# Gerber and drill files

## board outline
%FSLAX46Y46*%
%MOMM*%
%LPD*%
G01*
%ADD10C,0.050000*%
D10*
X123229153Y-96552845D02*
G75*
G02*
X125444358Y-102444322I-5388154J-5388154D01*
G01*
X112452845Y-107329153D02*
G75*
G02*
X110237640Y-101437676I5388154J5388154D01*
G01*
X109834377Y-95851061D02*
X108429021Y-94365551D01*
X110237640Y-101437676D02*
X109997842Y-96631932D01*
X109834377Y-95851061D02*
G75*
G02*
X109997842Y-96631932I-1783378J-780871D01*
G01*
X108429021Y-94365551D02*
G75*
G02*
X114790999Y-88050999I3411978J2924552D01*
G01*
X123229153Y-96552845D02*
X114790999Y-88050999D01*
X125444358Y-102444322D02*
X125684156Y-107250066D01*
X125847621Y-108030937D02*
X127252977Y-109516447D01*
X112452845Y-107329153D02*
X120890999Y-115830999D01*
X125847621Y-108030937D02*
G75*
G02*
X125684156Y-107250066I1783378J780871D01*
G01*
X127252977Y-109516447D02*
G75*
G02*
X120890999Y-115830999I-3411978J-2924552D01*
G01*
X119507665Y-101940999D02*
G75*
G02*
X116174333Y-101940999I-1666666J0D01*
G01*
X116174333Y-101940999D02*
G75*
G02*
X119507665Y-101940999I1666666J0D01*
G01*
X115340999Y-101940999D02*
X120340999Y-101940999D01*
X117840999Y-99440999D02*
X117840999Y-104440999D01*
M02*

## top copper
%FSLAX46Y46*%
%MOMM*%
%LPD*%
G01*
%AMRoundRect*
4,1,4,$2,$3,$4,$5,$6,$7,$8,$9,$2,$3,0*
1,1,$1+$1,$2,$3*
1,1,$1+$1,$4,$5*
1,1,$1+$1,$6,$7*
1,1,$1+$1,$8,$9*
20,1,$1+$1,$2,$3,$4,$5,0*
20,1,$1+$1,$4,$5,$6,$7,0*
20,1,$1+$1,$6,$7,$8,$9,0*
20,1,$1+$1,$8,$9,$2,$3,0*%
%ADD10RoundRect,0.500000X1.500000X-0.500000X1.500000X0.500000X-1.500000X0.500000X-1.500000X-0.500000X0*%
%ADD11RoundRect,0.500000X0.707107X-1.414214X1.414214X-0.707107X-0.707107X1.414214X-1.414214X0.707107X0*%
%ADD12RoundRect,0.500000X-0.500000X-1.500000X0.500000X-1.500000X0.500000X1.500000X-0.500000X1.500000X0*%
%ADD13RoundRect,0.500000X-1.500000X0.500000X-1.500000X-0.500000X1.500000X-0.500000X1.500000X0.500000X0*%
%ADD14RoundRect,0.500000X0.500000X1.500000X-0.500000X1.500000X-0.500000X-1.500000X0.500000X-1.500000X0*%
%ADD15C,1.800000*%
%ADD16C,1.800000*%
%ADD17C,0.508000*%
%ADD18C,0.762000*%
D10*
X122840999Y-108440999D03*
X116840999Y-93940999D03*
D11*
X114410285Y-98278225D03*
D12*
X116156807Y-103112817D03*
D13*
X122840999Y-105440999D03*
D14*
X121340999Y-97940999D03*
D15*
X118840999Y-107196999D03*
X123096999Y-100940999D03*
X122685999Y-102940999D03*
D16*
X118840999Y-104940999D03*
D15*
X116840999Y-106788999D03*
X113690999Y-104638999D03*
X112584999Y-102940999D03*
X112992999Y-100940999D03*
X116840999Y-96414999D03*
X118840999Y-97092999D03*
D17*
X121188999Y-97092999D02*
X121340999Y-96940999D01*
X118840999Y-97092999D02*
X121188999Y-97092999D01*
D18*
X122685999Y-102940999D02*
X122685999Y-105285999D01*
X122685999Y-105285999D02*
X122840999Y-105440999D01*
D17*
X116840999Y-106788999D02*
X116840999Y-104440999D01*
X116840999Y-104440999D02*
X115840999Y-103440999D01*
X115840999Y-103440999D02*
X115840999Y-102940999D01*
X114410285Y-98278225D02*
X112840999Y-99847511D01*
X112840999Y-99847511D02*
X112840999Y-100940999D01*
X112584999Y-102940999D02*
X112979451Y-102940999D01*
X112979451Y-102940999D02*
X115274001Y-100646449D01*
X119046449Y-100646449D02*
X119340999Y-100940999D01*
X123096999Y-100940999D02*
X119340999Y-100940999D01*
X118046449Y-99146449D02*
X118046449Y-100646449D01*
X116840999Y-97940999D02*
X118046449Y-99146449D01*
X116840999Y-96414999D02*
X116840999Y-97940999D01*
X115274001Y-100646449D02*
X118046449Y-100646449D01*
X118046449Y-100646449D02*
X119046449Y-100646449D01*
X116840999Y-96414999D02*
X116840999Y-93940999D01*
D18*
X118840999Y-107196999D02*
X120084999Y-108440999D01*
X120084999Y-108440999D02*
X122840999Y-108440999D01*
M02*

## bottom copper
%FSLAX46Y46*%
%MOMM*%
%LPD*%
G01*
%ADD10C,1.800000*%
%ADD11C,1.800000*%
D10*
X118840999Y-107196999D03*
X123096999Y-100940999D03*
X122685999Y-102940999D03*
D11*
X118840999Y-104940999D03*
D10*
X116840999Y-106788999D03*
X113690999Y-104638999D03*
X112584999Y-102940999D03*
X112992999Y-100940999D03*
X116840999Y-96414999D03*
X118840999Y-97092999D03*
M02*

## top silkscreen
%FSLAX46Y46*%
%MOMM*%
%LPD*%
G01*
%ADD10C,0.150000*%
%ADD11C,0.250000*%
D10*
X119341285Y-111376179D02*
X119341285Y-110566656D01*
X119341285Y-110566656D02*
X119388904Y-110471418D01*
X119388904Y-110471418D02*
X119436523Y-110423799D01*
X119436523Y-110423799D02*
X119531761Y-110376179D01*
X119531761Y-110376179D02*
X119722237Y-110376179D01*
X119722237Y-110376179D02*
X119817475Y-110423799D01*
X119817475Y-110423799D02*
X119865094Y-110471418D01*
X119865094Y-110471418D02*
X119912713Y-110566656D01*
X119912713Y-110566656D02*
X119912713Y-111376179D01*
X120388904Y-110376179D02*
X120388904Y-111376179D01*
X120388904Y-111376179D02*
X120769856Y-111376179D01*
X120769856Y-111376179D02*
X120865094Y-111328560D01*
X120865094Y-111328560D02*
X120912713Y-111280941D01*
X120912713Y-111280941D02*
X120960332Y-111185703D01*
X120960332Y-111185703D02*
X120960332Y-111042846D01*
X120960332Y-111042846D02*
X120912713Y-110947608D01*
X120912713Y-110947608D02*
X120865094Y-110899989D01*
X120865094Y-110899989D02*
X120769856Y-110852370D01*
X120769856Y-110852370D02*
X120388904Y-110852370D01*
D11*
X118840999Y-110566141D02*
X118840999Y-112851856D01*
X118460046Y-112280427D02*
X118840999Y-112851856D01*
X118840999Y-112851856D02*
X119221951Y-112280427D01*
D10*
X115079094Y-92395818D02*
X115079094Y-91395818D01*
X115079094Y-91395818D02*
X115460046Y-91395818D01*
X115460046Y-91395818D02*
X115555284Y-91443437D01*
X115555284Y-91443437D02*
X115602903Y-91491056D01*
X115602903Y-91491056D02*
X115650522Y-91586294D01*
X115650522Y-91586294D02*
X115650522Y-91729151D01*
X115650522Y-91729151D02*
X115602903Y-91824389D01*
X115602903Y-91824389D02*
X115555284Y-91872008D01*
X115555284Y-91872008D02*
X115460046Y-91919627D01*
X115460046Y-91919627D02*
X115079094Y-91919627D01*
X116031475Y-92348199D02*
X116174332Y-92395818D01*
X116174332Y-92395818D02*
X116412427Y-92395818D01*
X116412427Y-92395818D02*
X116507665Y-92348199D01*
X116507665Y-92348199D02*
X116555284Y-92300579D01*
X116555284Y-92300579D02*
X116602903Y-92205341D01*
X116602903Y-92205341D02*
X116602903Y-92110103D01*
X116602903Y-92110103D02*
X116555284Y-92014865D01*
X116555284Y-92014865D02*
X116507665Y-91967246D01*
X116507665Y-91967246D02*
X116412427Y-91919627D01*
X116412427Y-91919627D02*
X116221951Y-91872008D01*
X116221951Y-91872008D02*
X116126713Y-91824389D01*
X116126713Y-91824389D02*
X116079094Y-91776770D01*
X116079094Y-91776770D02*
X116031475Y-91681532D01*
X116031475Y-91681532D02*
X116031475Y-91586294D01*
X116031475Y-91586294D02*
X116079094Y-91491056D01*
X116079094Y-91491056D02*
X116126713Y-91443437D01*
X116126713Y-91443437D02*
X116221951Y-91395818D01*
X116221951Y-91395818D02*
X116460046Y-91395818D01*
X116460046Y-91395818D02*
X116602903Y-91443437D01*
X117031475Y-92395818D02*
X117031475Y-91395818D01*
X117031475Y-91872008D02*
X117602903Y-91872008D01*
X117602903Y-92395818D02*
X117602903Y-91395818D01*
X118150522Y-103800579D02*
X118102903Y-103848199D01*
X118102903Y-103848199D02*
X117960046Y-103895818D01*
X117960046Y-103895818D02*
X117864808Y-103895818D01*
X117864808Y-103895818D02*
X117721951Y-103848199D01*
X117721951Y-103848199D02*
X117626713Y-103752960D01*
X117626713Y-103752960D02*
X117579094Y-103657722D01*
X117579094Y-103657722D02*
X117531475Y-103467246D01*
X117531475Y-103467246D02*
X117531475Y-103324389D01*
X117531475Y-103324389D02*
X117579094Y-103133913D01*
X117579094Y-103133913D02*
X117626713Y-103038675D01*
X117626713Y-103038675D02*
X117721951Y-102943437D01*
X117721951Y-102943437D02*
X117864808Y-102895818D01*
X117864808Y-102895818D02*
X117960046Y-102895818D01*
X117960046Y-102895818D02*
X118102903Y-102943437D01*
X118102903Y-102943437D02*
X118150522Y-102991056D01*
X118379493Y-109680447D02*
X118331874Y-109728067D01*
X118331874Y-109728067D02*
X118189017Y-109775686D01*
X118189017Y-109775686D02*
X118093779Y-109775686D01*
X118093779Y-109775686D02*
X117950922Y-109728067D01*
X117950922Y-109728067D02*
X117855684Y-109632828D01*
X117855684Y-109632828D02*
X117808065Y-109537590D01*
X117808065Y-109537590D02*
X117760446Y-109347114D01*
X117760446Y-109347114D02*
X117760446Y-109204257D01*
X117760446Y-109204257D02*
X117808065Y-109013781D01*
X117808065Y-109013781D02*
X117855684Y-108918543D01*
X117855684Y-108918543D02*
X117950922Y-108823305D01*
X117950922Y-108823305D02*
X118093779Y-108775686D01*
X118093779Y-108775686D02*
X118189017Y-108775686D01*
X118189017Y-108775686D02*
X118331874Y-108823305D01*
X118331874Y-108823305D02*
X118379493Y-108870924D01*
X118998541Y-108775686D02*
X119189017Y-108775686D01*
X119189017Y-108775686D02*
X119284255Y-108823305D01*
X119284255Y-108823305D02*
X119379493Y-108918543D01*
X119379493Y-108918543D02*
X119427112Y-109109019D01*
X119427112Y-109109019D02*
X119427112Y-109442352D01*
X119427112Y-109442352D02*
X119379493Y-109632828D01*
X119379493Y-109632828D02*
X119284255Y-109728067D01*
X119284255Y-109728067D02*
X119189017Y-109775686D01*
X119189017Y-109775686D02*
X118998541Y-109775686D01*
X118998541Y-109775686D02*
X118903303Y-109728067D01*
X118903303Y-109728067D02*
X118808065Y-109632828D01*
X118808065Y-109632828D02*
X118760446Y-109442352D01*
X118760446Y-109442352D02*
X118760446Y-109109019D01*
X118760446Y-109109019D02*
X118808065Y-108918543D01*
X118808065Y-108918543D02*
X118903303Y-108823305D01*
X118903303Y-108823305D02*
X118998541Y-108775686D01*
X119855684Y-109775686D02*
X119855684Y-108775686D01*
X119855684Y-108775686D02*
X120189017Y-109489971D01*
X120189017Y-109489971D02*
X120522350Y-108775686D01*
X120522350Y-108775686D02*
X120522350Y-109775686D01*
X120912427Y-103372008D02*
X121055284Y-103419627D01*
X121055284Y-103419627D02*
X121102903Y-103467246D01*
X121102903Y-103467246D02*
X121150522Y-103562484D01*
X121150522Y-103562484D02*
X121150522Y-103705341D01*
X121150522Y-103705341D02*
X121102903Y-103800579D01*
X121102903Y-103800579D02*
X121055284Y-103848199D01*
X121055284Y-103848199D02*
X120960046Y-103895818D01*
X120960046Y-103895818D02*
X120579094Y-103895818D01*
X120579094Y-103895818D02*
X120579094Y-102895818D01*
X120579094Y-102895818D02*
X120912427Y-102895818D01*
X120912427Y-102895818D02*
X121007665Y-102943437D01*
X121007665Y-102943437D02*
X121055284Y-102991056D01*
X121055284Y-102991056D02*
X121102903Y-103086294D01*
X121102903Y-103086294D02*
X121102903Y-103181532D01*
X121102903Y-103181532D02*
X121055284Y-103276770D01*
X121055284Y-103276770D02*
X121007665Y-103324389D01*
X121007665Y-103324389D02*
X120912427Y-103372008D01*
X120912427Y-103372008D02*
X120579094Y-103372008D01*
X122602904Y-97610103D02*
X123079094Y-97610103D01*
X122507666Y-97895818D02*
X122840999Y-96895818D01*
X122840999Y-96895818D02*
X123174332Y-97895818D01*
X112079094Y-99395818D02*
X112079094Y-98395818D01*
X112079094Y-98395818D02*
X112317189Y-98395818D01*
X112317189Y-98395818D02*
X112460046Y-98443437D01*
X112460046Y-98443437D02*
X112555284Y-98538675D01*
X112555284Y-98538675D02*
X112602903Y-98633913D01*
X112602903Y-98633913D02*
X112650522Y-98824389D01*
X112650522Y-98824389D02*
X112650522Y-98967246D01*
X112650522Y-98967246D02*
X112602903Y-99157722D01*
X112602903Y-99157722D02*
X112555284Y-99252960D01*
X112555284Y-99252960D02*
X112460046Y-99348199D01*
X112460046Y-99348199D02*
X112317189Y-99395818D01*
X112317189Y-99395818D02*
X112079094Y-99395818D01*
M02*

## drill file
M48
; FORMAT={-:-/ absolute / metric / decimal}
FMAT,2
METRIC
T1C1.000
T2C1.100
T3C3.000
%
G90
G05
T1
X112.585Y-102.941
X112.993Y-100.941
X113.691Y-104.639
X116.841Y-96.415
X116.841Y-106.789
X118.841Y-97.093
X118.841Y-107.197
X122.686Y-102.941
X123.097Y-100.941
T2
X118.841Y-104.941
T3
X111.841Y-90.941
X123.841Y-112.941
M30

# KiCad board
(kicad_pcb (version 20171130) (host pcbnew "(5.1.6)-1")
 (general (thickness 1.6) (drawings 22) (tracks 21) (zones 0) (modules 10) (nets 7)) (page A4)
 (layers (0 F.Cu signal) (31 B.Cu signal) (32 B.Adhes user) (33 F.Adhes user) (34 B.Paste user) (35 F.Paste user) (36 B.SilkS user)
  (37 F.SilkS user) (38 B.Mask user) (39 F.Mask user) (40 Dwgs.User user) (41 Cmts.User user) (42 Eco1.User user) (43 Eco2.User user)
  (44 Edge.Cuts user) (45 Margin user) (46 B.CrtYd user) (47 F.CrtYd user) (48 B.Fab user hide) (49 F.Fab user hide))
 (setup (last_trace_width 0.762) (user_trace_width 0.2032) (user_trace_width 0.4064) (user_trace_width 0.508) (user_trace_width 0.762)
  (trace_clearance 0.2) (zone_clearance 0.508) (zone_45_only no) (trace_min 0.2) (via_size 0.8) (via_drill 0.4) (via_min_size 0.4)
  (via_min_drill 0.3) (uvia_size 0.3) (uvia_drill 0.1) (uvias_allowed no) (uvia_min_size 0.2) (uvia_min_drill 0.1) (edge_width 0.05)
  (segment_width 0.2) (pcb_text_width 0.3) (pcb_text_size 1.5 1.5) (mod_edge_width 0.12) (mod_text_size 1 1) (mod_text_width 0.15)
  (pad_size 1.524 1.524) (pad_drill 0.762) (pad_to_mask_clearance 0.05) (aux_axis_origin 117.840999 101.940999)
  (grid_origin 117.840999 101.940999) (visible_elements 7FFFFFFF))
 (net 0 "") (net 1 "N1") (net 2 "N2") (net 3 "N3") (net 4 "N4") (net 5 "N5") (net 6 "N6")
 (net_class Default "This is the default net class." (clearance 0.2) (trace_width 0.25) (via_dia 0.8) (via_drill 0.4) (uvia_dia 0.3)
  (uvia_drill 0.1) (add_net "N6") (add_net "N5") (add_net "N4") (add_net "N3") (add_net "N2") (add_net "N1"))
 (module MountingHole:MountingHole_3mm (layer B.Cu) (at 111.840999 90.940999 180)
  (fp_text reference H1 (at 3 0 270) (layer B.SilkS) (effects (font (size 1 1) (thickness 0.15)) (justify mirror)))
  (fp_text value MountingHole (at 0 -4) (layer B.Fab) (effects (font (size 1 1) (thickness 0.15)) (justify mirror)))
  (pad 1 np_thru_hole circle (at 0 0 180) (size 3 3) (drill 3) (layers *.Cu *.Mask)))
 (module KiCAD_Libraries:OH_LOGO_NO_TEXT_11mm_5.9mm (layer B.Cu) (at 118.340999 101.440999 200)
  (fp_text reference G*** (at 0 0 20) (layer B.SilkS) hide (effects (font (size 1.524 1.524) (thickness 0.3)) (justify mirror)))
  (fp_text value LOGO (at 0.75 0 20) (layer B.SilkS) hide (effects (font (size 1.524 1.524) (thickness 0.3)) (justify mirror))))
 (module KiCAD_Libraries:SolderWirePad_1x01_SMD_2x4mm (layer F.Cu) (at 122.840999 108.440999 90)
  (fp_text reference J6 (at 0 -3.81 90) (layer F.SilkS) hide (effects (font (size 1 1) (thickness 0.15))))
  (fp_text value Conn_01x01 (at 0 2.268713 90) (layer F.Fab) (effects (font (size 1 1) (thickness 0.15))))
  (pad 1 smd roundrect (at 0 0 90) (size 2 4) (layers F.Cu F.Paste F.Mask) (roundrect_rratio 0.25) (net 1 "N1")))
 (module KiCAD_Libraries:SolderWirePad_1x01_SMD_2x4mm (layer F.Cu) (at 116.840999 93.940999 90)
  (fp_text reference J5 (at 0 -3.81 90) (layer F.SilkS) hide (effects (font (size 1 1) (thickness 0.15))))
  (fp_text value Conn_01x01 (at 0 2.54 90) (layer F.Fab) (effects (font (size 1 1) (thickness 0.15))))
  (pad 1 smd roundrect (at 0 0 90) (size 2 4) (layers F.Cu F.Paste F.Mask) (roundrect_rratio 0.25) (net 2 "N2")))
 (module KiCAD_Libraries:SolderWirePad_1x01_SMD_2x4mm (layer F.Cu) (at 114.410285 98.278225 45)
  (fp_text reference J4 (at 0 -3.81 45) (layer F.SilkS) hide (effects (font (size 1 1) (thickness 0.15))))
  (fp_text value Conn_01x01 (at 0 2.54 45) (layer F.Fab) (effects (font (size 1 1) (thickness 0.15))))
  (pad 1 smd roundrect (at 0 0 45) (size 2 4) (layers F.Cu F.Paste F.Mask) (roundrect_rratio 0.25) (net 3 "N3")))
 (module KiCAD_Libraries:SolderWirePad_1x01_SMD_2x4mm (layer F.Cu) (at 116.156807 103.112817)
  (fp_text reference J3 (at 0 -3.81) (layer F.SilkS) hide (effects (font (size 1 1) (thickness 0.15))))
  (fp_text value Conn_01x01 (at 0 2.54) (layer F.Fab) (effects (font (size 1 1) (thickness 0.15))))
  (pad 1 smd roundrect (at 0 0) (size 2 4) (layers F.Cu F.Paste F.Mask) (roundrect_rratio 0.25) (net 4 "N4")))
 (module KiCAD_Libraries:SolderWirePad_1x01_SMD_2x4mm (layer F.Cu) (at 122.840999 105.440999 270)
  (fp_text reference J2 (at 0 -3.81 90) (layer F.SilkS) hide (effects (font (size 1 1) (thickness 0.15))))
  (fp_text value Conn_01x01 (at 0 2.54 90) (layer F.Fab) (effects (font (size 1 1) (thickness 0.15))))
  (pad 1 smd roundrect (at 0 0 270) (size 2 4) (layers F.Cu F.Paste F.Mask) (roundrect_rratio 0.25) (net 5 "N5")))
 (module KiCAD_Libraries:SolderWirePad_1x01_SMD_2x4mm (layer F.Cu) (at 121.340999 97.940999 180)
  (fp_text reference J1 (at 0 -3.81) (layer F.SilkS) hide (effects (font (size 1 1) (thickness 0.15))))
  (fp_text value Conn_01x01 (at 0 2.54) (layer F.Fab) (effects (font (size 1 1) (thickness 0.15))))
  (pad 1 smd roundrect (at 0 0 180) (size 2 4) (layers F.Cu F.Paste F.Mask) (roundrect_rratio 0.25) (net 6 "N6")))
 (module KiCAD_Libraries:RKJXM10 (layer B.Cu) (at 117.840999 101.940999)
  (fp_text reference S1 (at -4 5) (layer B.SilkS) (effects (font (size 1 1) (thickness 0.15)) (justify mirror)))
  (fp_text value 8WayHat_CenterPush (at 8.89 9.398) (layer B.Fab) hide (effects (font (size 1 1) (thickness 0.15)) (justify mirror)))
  (pad COM thru_hole circle (at 1 5.256) (size 1.8 1.8) (drill 1) (layers *.Cu *.Mask) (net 1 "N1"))
  (pad PUSH3 thru_hole circle (at 5.256 -1) (size 1.8 1.8) (drill 1) (layers *.Cu *.Mask) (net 2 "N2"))
  (pad B thru_hole circle (at 4.845 1) (size 1.8 1.8) (drill 1) (layers *.Cu *.Mask) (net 5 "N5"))
  (pad "" np_thru_hole circle (at 1 3) (size 1.8 1.8) (drill 1.1) (layers *.Cu *.Mask))
  (pad C thru_hole circle (at -1 4.848) (size 1.8 1.8) (drill 1) (layers *.Cu *.Mask) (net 4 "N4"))
  (pad GND thru_hole circle (at -4.15 2.698) (size 1.8 1.8) (drill 1) (layers *.Cu *.Mask))
  (pad PUSH1 thru_hole circle (at -5.256 1) (size 1.8 1.8) (drill 1) (layers *.Cu *.Mask) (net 2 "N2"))
  (pad D thru_hole circle (at -4.848 -1) (size 1.8 1.8) (drill 1) (layers *.Cu *.Mask) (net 3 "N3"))
  (pad PUSH2 thru_hole circle (at -1 -5.526) (size 1.8 1.8) (drill 1) (layers *.Cu *.Mask) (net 2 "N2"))
  (pad A thru_hole circle (at 1 -4.848) (size 1.8 1.8) (drill 1) (layers *.Cu *.Mask) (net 6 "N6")))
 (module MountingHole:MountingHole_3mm (layer B.Cu) (at 123.840999 112.940999)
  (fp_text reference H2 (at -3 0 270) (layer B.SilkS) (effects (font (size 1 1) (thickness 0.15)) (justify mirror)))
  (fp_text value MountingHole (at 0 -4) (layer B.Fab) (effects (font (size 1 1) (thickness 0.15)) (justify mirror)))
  (pad 1 np_thru_hole circle (at 0 0) (size 3 3) (drill 3) (layers *.Cu *.Mask)))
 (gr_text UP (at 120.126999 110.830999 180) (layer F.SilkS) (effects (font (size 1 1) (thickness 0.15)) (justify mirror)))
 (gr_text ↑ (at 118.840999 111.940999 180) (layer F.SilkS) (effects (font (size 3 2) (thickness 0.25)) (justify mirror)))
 (gr_arc (start 117.840999 101.940999) (end 125.444358 102.444322) (angle -48.787309) (layer Edge.Cuts) (width 0.05))
 (gr_arc (start 117.840999 101.940999) (end 110.23764 101.437676) (angle -48.787309) (layer Edge.Cuts) (width 0.05))
 (gr_line (start 109.834377 95.851061) (end 108.429021 94.365551) (layer Edge.Cuts) (width 0.05))
 (gr_line (start 110.23764 101.437676) (end 109.997842 96.631932) (layer Edge.Cuts) (width 0.05))
 (gr_arc (start 108.050999 96.631932) (end 109.997842 96.631932) (angle -23.64670356) (layer Edge.Cuts) (width 0.05))
 (gr_arc (start 111.840999 91.440999) (end 114.790999 88.050999) (angle -171.631297) (layer Edge.Cuts) (width 0.05))
 (gr_line (start 123.229153 96.552845) (end 114.790999 88.050999) (layer Edge.Cuts) (width 0.05))
 (gr_line (start 125.444358 102.444322) (end 125.684156 107.250066) (layer Edge.Cuts) (width 0.05))
 (gr_line (start 125.847621 108.030937) (end 127.252977 109.516447) (layer Edge.Cuts) (width 0.05))
 (gr_line (start 112.452845 107.329153) (end 120.890999 115.830999) (layer Edge.Cuts) (width 0.05))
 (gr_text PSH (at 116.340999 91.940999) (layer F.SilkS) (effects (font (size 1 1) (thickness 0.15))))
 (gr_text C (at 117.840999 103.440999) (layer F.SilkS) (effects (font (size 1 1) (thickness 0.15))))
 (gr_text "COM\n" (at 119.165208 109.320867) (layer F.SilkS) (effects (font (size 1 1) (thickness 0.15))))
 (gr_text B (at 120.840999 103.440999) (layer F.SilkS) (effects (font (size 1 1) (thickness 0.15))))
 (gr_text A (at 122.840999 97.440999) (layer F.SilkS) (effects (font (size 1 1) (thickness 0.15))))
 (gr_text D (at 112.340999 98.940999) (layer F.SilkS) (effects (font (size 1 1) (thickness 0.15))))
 (gr_arc (start 127.630999 107.250066) (end 125.684156 107.250066) (angle -23.64670356) (layer Edge.Cuts) (width 0.05))
 (gr_arc (start 123.840999 112.440999) (end 120.890999 115.830999) (angle -171.631297) (layer Edge.Cuts) (width 0.05))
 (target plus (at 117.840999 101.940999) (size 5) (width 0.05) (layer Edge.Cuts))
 (segment (start 121.188999 97.092999) (end 121.340999 96.940999) (width 0.508) (layer F.Cu) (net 6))
 (segment (start 118.840999 97.092999) (end 121.188999 97.092999) (width 0.508) (layer F.Cu) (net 6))
 (segment (start 122.685999 102.940999) (end 122.685999 105.285999) (width 0.762) (layer F.Cu) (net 5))
 (segment (start 122.685999 105.285999) (end 122.840999 105.440999) (width 0.762) (layer F.Cu) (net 5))
 (segment (start 116.840999 106.788999) (end 116.840999 104.440999) (width 0.508) (layer F.Cu) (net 4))
 (segment (start 116.840999 104.440999) (end 115.840999 103.440999) (width 0.508) (layer F.Cu) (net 4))
 (segment (start 115.840999 103.440999) (end 115.840999 102.940999) (width 0.508) (layer F.Cu) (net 4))
 (segment (start 114.410285 98.278225) (end 112.840999 99.847511) (width 0.508) (layer F.Cu) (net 3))
 (segment (start 112.840999 99.847511) (end 112.840999 100.940999) (width 0.508) (layer F.Cu) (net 3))
 (segment (start 112.584999 102.940999) (end 112.979451 102.940999) (width 0.508) (layer F.Cu) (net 2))
 (segment (start 112.979451 102.940999) (end 115.274001 100.646449) (width 0.508) (layer F.Cu) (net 2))
 (segment (start 119.046449 100.646449) (end 119.340999 100.940999) (width 0.508) (layer F.Cu) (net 2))
 (segment (start 123.096999 100.940999) (end 119.340999 100.940999) (width 0.508) (layer F.Cu) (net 2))
 (segment (start 118.046449 99.146449) (end 118.046449 100.646449) (width 0.508) (layer F.Cu) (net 2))
 (segment (start 116.840999 97.940999) (end 118.046449 99.146449) (width 0.508) (layer F.Cu) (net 2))
 (segment (start 116.840999 96.414999) (end 116.840999 97.940999) (width 0.508) (layer F.Cu) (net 2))
 (segment (start 115.274001 100.646449) (end 118.046449 100.646449) (width 0.508) (layer F.Cu) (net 2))
 (segment (start 118.046449 100.646449) (end 119.046449 100.646449) (width 0.508) (layer F.Cu) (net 2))
 (segment (start 116.840999 96.414999) (end 116.840999 93.940999) (width 0.508) (layer F.Cu) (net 2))
 (segment (start 118.840999 107.196999) (end 120.084999 108.440999) (width 0.762) (layer F.Cu) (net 1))
 (segment (start 120.084999 108.440999) (end 122.840999 108.440999) (width 0.762) (layer F.Cu) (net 1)))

